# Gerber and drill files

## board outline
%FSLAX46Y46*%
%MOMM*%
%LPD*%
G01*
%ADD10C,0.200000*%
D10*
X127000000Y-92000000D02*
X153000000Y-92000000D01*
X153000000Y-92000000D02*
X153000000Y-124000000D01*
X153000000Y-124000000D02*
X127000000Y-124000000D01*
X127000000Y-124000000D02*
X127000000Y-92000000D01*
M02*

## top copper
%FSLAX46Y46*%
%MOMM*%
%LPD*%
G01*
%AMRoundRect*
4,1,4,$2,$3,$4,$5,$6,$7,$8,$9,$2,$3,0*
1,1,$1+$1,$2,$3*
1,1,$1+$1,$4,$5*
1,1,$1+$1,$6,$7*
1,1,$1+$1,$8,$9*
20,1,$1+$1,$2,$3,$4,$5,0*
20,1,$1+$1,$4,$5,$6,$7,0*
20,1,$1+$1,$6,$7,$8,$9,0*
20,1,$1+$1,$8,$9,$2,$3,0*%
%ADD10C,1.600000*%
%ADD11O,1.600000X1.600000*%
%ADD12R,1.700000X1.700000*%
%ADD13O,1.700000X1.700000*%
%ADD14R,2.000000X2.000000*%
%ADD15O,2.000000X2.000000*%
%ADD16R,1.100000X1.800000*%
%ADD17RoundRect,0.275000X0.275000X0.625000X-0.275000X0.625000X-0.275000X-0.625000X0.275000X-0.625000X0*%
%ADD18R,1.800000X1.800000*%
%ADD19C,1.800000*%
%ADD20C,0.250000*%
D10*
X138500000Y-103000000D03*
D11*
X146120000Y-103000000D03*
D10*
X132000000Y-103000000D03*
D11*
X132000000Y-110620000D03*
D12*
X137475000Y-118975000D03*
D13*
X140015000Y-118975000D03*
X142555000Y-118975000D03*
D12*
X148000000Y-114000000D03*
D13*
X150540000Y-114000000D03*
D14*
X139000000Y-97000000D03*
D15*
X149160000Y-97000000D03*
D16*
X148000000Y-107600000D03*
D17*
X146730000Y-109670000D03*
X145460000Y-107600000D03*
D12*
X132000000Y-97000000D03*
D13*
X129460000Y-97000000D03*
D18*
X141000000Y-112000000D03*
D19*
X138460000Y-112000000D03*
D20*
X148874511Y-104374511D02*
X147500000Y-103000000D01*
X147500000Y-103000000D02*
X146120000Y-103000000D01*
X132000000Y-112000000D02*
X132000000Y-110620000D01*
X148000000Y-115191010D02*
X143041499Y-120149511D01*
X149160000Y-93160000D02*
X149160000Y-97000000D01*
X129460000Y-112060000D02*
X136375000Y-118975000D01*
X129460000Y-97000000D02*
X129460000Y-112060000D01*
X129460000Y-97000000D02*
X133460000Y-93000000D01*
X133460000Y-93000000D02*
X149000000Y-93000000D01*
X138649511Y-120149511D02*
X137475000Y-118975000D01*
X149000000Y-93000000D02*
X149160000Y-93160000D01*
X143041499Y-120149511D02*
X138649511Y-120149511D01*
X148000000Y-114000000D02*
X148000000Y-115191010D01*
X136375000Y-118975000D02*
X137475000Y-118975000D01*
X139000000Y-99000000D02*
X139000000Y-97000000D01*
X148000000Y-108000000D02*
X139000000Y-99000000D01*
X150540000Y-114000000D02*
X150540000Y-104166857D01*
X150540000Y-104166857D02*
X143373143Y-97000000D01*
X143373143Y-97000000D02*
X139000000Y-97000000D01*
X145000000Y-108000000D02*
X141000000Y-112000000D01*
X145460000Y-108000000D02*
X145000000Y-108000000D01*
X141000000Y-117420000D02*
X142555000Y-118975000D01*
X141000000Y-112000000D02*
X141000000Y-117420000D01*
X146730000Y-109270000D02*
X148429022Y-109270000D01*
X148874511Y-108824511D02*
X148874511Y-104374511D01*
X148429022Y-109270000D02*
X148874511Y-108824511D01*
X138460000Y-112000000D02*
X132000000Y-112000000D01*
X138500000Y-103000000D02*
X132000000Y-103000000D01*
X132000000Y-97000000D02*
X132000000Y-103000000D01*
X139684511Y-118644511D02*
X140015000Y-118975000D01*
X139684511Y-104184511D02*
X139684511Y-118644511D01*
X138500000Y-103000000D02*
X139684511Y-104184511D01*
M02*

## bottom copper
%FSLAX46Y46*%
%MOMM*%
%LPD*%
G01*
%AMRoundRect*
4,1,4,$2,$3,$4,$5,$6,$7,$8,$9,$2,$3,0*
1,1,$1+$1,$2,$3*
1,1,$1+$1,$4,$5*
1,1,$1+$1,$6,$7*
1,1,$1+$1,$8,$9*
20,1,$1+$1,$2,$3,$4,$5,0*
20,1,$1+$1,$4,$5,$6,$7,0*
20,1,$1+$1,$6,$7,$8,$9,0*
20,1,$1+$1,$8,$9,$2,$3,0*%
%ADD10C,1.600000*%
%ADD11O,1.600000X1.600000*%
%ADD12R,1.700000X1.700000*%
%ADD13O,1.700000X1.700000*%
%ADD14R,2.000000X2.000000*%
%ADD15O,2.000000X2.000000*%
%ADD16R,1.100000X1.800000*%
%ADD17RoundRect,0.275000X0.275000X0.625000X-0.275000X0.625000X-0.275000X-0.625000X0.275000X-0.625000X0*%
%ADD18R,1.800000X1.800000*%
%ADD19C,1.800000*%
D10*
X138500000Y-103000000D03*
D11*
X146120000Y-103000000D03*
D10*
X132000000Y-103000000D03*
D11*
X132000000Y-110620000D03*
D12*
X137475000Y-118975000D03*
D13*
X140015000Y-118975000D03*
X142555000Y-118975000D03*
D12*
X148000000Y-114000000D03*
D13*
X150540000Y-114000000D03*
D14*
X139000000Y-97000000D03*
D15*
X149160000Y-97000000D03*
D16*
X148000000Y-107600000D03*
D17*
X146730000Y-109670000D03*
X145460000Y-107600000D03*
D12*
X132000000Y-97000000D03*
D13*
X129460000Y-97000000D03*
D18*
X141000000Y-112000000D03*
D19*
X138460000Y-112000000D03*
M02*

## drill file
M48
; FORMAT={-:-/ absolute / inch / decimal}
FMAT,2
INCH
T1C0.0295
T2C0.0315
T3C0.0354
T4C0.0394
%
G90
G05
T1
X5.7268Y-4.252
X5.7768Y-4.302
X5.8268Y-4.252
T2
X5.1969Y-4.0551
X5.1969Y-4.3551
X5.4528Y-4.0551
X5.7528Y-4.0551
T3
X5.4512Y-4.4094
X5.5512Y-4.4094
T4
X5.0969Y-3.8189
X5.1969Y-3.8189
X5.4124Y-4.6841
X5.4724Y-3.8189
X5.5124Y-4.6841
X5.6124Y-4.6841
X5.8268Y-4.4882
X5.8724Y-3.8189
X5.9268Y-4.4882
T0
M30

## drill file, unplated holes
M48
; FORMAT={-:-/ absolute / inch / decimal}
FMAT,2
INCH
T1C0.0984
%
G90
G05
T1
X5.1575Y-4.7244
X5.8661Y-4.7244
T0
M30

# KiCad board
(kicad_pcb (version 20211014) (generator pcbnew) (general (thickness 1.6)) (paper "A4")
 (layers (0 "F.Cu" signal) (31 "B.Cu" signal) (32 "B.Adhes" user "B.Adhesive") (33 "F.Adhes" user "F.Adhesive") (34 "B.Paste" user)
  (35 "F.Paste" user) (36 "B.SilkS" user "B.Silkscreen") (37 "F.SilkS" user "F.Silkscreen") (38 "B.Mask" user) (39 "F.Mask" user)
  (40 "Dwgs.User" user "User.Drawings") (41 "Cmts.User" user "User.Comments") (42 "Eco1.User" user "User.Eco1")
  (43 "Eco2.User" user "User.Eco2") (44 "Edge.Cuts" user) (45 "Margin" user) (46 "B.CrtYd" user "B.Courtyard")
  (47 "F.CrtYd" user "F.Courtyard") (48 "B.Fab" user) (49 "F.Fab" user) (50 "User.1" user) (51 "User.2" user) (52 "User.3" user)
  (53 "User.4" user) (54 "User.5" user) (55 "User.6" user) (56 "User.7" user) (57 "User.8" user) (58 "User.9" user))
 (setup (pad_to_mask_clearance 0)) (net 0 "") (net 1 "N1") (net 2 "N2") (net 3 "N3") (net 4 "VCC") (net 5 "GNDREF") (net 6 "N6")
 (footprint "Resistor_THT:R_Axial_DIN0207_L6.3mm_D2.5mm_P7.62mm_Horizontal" (layer "F.Cu") (at 138.5 103)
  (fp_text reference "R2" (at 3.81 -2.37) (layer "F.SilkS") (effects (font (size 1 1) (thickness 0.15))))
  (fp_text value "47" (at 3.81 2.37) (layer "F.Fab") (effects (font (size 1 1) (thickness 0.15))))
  (pad "1" thru_hole circle (at 0 0) (size 1.6 1.6) (drill 0.8) (layers *.Cu *.Mask) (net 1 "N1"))
  (pad "2" thru_hole oval (at 7.62 0) (size 1.6 1.6) (drill 0.8) (layers *.Cu *.Mask) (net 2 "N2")))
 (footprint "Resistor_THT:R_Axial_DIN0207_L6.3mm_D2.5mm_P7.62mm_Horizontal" (layer "F.Cu") (at 132 103 -90)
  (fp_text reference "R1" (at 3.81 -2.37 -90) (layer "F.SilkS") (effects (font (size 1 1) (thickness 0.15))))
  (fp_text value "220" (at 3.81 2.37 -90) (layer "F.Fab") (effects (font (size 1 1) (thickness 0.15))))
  (pad "1" thru_hole circle (at 0 0 270) (size 1.6 1.6) (drill 0.8) (layers *.Cu *.Mask) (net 1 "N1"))
  (pad "2" thru_hole oval (at 7.62 0 270) (size 1.6 1.6) (drill 0.8) (layers *.Cu *.Mask) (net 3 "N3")))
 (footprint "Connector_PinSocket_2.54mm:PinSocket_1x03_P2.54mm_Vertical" (layer "F.Cu") (at 137.475 118.975 90)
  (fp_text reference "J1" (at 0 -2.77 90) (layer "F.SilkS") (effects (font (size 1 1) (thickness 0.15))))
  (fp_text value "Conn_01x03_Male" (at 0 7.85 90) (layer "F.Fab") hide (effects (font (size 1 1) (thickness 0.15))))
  (pad "1" thru_hole rect (at 0 0 90) (size 1.7 1.7) (drill 1) (layers *.Cu *.Mask) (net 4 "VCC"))
  (pad "2" thru_hole oval (at 0 2.54 90) (size 1.7 1.7) (drill 1) (layers *.Cu *.Mask) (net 1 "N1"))
  (pad "3" thru_hole oval (at 0 5.08 90) (size 1.7 1.7) (drill 1) (layers *.Cu *.Mask) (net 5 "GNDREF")))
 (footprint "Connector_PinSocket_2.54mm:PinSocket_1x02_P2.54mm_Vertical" (layer "F.Cu") (at 148 114 90)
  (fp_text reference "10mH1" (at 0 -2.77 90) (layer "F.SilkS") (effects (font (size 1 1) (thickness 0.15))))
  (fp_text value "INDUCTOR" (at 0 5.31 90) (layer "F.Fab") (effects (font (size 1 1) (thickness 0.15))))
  (pad "1" thru_hole rect (at 0 0 90) (size 1.7 1.7) (drill 1) (layers *.Cu *.Mask) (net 4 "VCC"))
  (pad "2" thru_hole oval (at 0 2.54 90) (size 1.7 1.7) (drill 1) (layers *.Cu *.Mask) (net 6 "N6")))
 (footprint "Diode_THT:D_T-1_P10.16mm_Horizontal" (layer "F.Cu") (at 139 97)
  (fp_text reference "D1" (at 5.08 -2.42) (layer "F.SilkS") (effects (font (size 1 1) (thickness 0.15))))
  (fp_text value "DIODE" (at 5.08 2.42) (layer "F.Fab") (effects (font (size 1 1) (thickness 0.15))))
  (pad "1" thru_hole rect (at 0 0) (size 2 2) (drill 1) (layers *.Cu *.Mask) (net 6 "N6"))
  (pad "2" thru_hole oval (at 10.16 0) (size 2 2) (drill 1) (layers *.Cu *.Mask) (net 4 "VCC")))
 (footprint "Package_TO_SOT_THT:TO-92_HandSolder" (layer "F.Cu") (at 148 108 180)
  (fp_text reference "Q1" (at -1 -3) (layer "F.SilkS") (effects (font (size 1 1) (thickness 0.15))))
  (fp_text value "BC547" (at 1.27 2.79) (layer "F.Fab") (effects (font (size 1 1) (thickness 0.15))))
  (pad "1" thru_hole rect (at 0 0 180) (size 1.1 1.8) (drill 0.75 (offset 0 0.4)) (layers *.Cu *.Mask) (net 6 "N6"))
  (pad "2" thru_hole roundrect (at 1.27 -1.27 180) (size 1.1 1.8) (drill 0.75 (offset 0 -0.4)) (layers *.Cu *.Mask) (roundrect_rratio 0.25)
   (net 2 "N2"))
  (pad "3" thru_hole roundrect (at 2.54 0 180) (size 1.1 1.8) (drill 0.75 (offset 0 0.4)) (layers *.Cu *.Mask) (roundrect_rratio 0.25)
   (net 5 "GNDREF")))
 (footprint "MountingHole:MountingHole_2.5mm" (layer "F.Cu") (at 149 120)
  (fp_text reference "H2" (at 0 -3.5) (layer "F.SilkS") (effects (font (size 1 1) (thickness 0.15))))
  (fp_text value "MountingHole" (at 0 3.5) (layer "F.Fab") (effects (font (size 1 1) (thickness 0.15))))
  (pad "" np_thru_hole circle (at 0 0) (size 2.5 2.5) (drill 2.5) (layers *.Cu *.Mask)))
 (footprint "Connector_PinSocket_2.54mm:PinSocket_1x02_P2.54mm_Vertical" (layer "F.Cu") (at 132 97 -90)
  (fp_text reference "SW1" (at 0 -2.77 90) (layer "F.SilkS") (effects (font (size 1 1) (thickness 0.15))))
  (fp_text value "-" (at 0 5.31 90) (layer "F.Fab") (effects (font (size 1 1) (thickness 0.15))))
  (pad "1" thru_hole rect (at 0 0 270) (size 1.7 1.7) (drill 1) (layers *.Cu *.Mask) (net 1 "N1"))
  (pad "2" thru_hole oval (at 0 2.54 270) (size 1.7 1.7) (drill 1) (layers *.Cu *.Mask) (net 4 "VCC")))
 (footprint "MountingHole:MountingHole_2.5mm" (layer "F.Cu") (at 131 120)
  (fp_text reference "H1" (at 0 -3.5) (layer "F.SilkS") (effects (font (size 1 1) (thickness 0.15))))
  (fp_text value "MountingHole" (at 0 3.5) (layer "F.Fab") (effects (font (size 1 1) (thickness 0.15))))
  (pad "" np_thru_hole circle (at 0 0) (size 2.5 2.5) (drill 2.5) (layers *.Cu *.Mask)))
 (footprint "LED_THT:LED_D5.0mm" (layer "F.Cu") (at 141 112 180)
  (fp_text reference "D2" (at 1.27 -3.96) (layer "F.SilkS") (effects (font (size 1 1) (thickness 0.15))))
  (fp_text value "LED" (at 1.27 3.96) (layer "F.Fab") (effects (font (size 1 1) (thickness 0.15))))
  (pad "1" thru_hole rect (at 0 0 180) (size 1.8 1.8) (drill 0.9) (layers *.Cu *.Mask) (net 5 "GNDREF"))
  (pad "2" thru_hole circle (at 2.54 0 180) (size 1.8 1.8) (drill 0.9) (layers *.Cu *.Mask) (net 3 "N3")))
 (gr_rect (start 127 92) (end 153 124) (layer "Edge.Cuts") (width 0.2) (fill none))
 (segment (start 148 115.19101) (end 143.041499 120.149511) (width 0.25) (layer "F.Cu") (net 4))
 (segment (start 149.16 93.16) (end 149.16 97) (width 0.25) (layer "F.Cu") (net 4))
 (segment (start 129.46 112.06) (end 136.375 118.975) (width 0.25) (layer "F.Cu") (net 4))
 (segment (start 129.46 97) (end 129.46 112.06) (width 0.25) (layer "F.Cu") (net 4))
 (segment (start 129.46 97) (end 133.46 93) (width 0.25) (layer "F.Cu") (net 4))
 (segment (start 133.46 93) (end 149 93) (width 0.25) (layer "F.Cu") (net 4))
 (segment (start 138.649511 120.149511) (end 137.475 118.975) (width 0.25) (layer "F.Cu") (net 4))
 (segment (start 149 93) (end 149.16 93.16) (width 0.25) (layer "F.Cu") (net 4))
 (segment (start 143.041499 120.149511) (end 138.649511 120.149511) (width 0.25) (layer "F.Cu") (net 4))
 (segment (start 148 114) (end 148 115.19101) (width 0.25) (layer "F.Cu") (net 4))
 (segment (start 136.375 118.975) (end 137.475 118.975) (width 0.25) (layer "F.Cu") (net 4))
 (segment (start 139 99) (end 139 97) (width 0.25) (layer "F.Cu") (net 6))
 (segment (start 148 108) (end 139 99) (width 0.25) (layer "F.Cu") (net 6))
 (segment (start 150.54 114) (end 150.54 104.166857) (width 0.25) (layer "F.Cu") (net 6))
 (segment (start 150.54 104.166857) (end 143.373143 97) (width 0.25) (layer "F.Cu") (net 6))
 (segment (start 143.373143 97) (end 139 97) (width 0.25) (layer "F.Cu") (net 6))
 (segment (start 145 108) (end 141 112) (width 0.25) (layer "F.Cu") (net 5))
 (segment (start 145.46 108) (end 145 108) (width 0.25) (layer "F.Cu") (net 5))
 (segment (start 141 117.42) (end 142.555 118.975) (width 0.25) (layer "F.Cu") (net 5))
 (segment (start 141 112) (end 141 117.42) (width 0.25) (layer "F.Cu") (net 5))
 (segment (start 147.5 103) (end 146.12 103) (width 0.25) (layer "F.Cu") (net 2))
 (segment (start 146.73 109.27) (end 148.429022 109.27) (width 0.25) (layer "F.Cu") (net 2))
 (segment (start 148.874511 108.824511) (end 148.874511 104.374511) (width 0.25) (layer "F.Cu") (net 2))
 (segment (start 148.874511 104.374511) (end 147.5 103) (width 0.25) (layer "F.Cu") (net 2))
 (segment (start 148.429022 109.27) (end 148.874511 108.824511) (width 0.25) (layer "F.Cu") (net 2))
 (segment (start 138.46 112) (end 132 112) (width 0.25) (layer "F.Cu") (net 3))
 (segment (start 132 112) (end 132 110.62) (width 0.25) (layer "F.Cu") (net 3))
 (segment (start 138.5 103) (end 132 103) (width 0.25) (layer "F.Cu") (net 1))
 (segment (start 132 97) (end 132 103) (width 0.25) (layer "F.Cu") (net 1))
 (segment (start 139.684511 118.644511) (end 140.015 118.975) (width 0.25) (layer "F.Cu") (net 1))
 (segment (start 139.684511 104.184511) (end 139.684511 118.644511) (width 0.25) (layer "F.Cu") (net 1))
 (segment (start 138.5 103) (end 139.684511 104.184511) (width 0.25) (layer "F.Cu") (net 1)))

